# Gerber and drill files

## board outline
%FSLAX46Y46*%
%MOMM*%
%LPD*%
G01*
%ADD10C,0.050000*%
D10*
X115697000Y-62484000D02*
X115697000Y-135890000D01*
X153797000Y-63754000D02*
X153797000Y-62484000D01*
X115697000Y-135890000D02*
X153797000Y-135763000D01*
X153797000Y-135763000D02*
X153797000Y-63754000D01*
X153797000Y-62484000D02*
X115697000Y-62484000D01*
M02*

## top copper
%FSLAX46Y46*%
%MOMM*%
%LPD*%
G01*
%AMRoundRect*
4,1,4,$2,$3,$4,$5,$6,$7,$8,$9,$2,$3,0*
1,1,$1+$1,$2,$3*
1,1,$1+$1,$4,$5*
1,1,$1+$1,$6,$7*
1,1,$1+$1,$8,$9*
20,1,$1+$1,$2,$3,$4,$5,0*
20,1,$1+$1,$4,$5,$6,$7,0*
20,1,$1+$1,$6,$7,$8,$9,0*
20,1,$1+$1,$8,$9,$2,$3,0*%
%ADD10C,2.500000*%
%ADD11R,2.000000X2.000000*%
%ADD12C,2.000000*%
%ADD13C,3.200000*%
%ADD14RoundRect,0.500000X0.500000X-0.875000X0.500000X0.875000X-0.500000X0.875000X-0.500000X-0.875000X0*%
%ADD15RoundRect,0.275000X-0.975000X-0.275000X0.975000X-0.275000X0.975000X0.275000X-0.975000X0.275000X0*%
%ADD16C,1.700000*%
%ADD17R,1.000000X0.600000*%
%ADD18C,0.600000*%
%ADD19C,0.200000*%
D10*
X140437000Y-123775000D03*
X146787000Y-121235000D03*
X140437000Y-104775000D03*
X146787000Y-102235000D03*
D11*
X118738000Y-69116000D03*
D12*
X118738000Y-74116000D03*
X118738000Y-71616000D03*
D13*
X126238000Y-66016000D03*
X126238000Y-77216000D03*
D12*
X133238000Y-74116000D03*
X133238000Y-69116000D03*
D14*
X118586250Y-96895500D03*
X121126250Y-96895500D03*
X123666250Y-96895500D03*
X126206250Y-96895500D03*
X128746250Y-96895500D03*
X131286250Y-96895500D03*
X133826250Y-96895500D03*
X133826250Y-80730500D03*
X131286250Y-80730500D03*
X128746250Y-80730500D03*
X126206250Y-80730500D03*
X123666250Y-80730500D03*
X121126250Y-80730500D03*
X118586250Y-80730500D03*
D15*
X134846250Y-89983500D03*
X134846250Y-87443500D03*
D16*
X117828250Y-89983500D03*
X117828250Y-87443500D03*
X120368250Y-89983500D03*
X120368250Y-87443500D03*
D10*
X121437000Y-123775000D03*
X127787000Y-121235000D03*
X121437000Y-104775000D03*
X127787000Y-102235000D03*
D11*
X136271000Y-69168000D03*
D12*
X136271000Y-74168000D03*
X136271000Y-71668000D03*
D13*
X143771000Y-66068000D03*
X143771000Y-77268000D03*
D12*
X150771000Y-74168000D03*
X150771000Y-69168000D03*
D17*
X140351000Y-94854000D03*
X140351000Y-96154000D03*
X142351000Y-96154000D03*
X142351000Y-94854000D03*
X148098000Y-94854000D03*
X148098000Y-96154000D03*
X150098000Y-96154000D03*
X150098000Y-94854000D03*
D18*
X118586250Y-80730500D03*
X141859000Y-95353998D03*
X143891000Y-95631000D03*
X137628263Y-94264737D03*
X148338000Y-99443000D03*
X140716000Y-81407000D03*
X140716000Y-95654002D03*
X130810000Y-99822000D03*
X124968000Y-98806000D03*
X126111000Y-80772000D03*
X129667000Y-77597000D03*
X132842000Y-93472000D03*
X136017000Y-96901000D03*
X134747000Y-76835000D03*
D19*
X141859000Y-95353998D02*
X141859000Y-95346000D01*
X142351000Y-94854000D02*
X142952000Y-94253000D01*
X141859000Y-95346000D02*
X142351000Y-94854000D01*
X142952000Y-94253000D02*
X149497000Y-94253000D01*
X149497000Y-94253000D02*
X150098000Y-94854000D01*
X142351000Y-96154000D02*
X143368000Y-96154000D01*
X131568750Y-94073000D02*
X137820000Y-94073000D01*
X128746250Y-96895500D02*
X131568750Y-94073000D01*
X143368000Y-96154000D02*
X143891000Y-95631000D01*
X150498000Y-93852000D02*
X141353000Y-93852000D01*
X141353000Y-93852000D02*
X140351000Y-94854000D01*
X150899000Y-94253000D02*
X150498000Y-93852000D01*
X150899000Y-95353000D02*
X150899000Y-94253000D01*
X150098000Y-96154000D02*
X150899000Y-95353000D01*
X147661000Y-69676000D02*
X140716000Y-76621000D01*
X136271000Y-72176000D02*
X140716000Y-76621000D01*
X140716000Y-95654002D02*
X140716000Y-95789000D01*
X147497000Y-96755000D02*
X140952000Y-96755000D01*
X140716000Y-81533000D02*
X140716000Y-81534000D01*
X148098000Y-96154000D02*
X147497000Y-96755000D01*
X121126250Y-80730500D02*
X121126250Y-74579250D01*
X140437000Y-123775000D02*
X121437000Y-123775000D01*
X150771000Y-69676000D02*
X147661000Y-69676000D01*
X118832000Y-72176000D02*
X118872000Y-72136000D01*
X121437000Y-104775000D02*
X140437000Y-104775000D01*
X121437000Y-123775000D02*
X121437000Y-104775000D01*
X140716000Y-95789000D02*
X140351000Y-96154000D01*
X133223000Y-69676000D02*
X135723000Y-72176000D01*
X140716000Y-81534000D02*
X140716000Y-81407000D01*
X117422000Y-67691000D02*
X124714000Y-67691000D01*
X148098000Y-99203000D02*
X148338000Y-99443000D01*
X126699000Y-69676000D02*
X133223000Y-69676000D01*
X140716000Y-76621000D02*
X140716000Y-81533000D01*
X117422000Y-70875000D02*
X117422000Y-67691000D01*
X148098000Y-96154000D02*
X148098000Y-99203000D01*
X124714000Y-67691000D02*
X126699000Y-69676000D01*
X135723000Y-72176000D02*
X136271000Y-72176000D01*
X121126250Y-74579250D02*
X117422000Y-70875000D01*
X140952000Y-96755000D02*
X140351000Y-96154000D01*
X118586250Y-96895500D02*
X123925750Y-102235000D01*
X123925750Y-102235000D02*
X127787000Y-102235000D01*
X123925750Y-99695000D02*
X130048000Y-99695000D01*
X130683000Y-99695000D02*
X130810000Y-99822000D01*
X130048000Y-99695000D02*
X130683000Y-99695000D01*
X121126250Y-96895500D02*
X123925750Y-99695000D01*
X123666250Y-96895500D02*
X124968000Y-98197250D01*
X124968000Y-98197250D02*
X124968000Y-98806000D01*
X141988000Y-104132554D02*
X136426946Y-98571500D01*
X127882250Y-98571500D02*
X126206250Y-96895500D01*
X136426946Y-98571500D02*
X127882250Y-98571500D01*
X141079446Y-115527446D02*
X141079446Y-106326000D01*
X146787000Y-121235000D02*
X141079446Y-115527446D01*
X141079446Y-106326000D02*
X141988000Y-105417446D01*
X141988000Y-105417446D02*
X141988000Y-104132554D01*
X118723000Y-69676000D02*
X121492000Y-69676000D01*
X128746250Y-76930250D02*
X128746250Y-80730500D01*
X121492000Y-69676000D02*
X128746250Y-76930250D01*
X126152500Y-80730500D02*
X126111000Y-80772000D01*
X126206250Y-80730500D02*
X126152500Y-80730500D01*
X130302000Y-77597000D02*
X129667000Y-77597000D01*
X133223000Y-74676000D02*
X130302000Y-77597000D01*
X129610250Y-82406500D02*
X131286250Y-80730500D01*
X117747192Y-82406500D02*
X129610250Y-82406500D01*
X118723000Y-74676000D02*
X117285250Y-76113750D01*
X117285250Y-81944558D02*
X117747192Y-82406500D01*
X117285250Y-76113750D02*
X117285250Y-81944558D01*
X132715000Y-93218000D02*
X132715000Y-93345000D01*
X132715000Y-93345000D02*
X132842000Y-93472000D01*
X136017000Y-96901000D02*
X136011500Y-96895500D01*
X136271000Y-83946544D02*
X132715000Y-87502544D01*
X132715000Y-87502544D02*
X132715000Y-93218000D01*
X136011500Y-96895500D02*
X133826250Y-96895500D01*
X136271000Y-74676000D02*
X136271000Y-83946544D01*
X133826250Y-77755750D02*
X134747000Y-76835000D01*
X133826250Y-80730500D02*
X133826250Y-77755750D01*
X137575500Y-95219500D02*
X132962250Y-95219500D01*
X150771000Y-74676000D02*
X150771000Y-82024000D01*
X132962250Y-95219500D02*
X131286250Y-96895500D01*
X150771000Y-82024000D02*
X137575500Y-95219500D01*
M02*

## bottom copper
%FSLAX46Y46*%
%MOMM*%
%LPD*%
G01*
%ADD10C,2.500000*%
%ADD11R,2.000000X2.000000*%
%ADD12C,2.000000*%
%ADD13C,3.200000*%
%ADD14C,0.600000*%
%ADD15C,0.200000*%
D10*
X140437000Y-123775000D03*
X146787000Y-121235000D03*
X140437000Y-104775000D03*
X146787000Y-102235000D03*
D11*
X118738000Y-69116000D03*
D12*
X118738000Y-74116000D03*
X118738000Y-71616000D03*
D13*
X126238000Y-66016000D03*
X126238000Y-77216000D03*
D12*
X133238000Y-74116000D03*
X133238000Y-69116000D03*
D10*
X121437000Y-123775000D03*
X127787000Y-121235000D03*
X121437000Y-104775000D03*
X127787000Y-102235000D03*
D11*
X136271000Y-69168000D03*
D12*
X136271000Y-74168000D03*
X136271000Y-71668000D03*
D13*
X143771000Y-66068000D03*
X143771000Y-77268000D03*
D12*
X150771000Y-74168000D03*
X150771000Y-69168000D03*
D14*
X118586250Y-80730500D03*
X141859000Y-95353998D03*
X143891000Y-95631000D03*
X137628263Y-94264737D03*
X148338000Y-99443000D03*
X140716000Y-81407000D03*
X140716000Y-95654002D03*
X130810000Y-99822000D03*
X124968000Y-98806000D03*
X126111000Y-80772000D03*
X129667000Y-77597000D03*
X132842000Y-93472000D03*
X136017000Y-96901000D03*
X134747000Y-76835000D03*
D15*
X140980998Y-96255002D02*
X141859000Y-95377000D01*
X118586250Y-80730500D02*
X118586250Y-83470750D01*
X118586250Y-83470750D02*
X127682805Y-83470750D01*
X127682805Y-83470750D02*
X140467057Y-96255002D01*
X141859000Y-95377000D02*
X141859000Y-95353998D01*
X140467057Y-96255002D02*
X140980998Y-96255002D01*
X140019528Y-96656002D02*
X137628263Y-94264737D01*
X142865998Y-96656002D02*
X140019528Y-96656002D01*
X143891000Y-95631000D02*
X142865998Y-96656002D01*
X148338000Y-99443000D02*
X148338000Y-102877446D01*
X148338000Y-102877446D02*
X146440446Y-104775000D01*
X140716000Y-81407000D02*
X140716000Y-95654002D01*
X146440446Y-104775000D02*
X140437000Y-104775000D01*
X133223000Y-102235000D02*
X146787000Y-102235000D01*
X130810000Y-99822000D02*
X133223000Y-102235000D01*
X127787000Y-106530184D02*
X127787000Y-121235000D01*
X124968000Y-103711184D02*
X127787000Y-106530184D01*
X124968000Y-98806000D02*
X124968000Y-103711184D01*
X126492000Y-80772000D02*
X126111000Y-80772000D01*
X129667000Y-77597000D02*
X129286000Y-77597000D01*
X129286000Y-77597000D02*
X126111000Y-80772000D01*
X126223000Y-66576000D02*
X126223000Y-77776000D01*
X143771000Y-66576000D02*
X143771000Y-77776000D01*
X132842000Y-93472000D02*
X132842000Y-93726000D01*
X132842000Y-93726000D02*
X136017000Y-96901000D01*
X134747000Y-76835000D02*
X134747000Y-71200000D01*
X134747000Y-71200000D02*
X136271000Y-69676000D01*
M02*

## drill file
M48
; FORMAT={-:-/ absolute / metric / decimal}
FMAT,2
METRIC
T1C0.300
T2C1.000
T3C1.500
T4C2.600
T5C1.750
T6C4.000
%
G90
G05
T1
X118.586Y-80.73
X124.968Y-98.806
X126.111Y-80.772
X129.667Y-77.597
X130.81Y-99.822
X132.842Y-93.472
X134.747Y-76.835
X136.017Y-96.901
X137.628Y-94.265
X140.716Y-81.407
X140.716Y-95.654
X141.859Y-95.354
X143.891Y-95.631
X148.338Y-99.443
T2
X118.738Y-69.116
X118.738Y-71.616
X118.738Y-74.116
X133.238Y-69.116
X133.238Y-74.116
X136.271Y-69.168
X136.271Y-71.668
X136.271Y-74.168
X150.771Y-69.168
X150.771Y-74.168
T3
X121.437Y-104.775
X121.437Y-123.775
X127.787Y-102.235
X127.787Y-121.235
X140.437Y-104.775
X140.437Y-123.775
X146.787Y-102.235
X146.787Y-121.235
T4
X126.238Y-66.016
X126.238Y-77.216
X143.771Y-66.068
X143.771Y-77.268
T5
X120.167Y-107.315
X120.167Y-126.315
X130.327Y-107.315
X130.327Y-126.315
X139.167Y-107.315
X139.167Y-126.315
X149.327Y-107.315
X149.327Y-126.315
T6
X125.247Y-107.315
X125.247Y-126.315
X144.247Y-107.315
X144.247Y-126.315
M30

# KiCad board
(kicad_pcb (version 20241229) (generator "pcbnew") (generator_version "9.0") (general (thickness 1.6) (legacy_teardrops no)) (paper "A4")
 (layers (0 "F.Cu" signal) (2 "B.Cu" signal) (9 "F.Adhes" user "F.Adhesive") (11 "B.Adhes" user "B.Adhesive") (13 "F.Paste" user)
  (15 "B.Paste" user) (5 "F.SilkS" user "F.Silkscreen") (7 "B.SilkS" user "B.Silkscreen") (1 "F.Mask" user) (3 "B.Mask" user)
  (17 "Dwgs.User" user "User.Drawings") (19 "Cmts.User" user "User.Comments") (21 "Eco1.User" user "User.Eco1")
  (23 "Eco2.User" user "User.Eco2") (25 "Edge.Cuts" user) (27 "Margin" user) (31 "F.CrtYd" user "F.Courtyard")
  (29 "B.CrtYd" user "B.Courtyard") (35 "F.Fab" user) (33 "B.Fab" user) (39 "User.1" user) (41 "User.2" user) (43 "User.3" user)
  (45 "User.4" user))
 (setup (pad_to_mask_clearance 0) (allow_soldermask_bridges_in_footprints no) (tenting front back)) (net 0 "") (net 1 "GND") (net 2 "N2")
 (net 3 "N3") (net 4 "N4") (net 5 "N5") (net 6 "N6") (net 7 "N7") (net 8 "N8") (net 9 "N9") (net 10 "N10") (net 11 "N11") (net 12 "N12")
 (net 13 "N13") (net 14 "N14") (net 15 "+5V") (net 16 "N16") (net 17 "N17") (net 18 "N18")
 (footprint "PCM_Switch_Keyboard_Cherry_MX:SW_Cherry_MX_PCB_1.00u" (layer "F.Cu") (at 144.247 126.315)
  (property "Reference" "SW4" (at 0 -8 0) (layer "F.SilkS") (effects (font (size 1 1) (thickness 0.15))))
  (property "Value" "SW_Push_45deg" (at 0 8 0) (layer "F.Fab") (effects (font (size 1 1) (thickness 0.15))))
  (pad "" np_thru_hole circle (at -5.08 0) (size 1.75 1.75) (drill 1.75) (layers "*.Cu" "*.Mask"))
  (pad "" np_thru_hole circle (at 0 0) (size 4 4) (drill 4) (layers "*.Cu" "*.Mask"))
  (pad "" np_thru_hole circle (at 5.08 0) (size 1.75 1.75) (drill 1.75) (layers "*.Cu" "*.Mask"))
  (pad "1" thru_hole circle (at -3.81 -2.54) (size 2.5 2.5) (drill 1.5) (layers "*.Cu" "*.Mask") (remove_unused_layers no) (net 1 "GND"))
  (pad "2" thru_hole circle (at 2.54 -5.08) (size 2.5 2.5) (drill 1.5) (layers "*.Cu" "*.Mask") (remove_unused_layers no) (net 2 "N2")))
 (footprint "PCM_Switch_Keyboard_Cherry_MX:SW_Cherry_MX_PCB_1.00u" (layer "F.Cu") (at 144.247 107.315)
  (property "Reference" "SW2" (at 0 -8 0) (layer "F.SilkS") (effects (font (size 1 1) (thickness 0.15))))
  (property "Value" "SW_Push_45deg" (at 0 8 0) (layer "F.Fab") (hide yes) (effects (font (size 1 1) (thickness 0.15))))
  (pad "" np_thru_hole circle (at -5.08 0) (size 1.75 1.75) (drill 1.75) (layers "*.Cu" "*.Mask"))
  (pad "" np_thru_hole circle (at 0 0) (size 4 4) (drill 4) (layers "*.Cu" "*.Mask"))
  (pad "" np_thru_hole circle (at 5.08 0) (size 1.75 1.75) (drill 1.75) (layers "*.Cu" "*.Mask"))
  (pad "1" thru_hole circle (at -3.81 -2.54) (size 2.5 2.5) (drill 1.5) (layers "*.Cu" "*.Mask") (remove_unused_layers no) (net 1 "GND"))
  (pad "2" thru_hole circle (at 2.54 -5.08) (size 2.5 2.5) (drill 1.5) (layers "*.Cu" "*.Mask") (remove_unused_layers no) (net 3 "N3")))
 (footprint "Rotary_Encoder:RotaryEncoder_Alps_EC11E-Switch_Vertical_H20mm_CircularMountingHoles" (layer "F.Cu") (at 118.738 69.116)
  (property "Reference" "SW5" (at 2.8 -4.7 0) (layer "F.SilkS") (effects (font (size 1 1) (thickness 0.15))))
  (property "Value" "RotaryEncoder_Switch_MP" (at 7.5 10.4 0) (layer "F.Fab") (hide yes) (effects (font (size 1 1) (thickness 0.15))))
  (pad "A" thru_hole rect (at 0 0) (size 2 2) (drill 1) (layers "*.Cu" "*.Mask") (remove_unused_layers no) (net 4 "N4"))
  (pad "B" thru_hole circle (at 0 5) (size 2 2) (drill 1) (layers "*.Cu" "*.Mask") (remove_unused_layers no) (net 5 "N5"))
  (pad "C" thru_hole circle (at 0 2.5) (size 2 2) (drill 1) (layers "*.Cu" "*.Mask") (remove_unused_layers no) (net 1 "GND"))
  (pad "MP" thru_hole circle (at 7.5 -3.1) (size 3.2 3.2) (drill 2.6) (layers "*.Cu" "*.Mask") (remove_unused_layers no) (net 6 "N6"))
  (pad "MP" thru_hole circle (at 7.5 8.1) (size 3.2 3.2) (drill 2.6) (layers "*.Cu" "*.Mask") (remove_unused_layers no) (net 6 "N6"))
  (pad "S1" thru_hole circle (at 14.5 5) (size 2 2) (drill 1) (layers "*.Cu" "*.Mask") (remove_unused_layers no) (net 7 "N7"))
  (pad "S2" thru_hole circle (at 14.5 0) (size 2 2) (drill 1) (layers "*.Cu" "*.Mask") (remove_unused_layers no) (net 1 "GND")))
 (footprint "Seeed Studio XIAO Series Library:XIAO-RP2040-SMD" (layer "F.Cu") (at 126.20625 88.8955 90)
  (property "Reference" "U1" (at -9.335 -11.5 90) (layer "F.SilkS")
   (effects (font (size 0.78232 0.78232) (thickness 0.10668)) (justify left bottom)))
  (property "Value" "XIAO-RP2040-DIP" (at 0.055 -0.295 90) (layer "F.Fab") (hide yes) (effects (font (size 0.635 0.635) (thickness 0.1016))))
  (pad "1" smd roundrect (at -8 -7.62 90) (size 2.75 2) (layers "F.Cu" "F.Mask" "F.Paste") (roundrect_rratio 0.25) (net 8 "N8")
   (solder_mask_margin 0.0508) (thermal_bridge_angle 45))
  (pad "2" smd roundrect (at -8 -5.08 90) (size 2.75 2) (layers "F.Cu" "F.Mask" "F.Paste") (roundrect_rratio 0.25) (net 3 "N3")
   (solder_mask_margin 0.0508) (thermal_bridge_angle 45))
  (pad "3" smd roundrect (at -8 -2.54 90) (size 2.75 2) (layers "F.Cu" "F.Mask" "F.Paste") (roundrect_rratio 0.25) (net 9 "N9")
   (solder_mask_margin 0.0508) (thermal_bridge_angle 45))
  (pad "4" smd roundrect (at -8 0 90) (size 2.75 2) (layers "F.Cu" "F.Mask" "F.Paste") (roundrect_rratio 0.25) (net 2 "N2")
   (solder_mask_margin 0.0508) (thermal_bridge_angle 45))
  (pad "5" smd roundrect (at -8 2.54 90) (size 2.75 2) (layers "F.Cu" "F.Mask" "F.Paste") (roundrect_rratio 0.25) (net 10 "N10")
   (solder_mask_margin 0.0508) (thermal_bridge_angle 45))
  (pad "6" smd roundrect (at -8 5.08 90) (size 2.75 2) (layers "F.Cu" "F.Mask" "F.Paste") (roundrect_rratio 0.25) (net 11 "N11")
   (solder_mask_margin 0.0508) (thermal_bridge_angle 45))
  (pad "7" smd roundrect (at -8 7.62 90) (size 2.75 2) (layers "F.Cu" "F.Mask" "F.Paste") (roundrect_rratio 0.25) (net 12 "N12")
   (solder_mask_margin 0.0508) (thermal_bridge_angle 45))
  (pad "8" smd roundrect (at 8.165 7.62 90) (size 2.75 2) (layers "F.Cu" "F.Mask" "F.Paste") (roundrect_rratio 0.25) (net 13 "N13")
   (solder_mask_margin 0.0508) (thermal_bridge_angle 45))
  (pad "9" smd roundrect (at 8.165 5.08 90) (size 2.75 2) (layers "F.Cu" "F.Mask" "F.Paste") (roundrect_rratio 0.25) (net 5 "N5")
   (solder_mask_margin 0.0508) (thermal_bridge_angle 45))
  (pad "10" smd roundrect (at 8.165 2.54 90) (size 2.75 2) (layers "F.Cu" "F.Mask" "F.Paste") (roundrect_rratio 0.25) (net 4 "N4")
   (solder_mask_margin 0.0508) (thermal_bridge_angle 45))
  (pad "11" smd roundrect (at 8.165 0 90) (size 2.75 2) (layers "F.Cu" "F.Mask" "F.Paste") (roundrect_rratio 0.25) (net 7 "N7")
   (solder_mask_margin 0.0508) (thermal_bridge_angle 45))
  (pad "12" smd roundrect (at 8.165 -2.54 90) (size 2.75 2) (layers "F.Cu" "F.Mask" "F.Paste") (roundrect_rratio 0.25) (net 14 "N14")
   (solder_mask_margin 0.0508) (thermal_bridge_angle 45))
  (pad "13" smd roundrect (at 8.165 -5.08 90) (size 2.75 2) (layers "F.Cu" "F.Mask" "F.Paste") (roundrect_rratio 0.25) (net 1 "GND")
   (solder_mask_margin 0.0508) (thermal_bridge_angle 45))
  (pad "14" smd roundrect (at 8.165 -7.62 90) (size 2.75 2) (layers "F.Cu" "F.Mask" "F.Paste") (roundrect_rratio 0.25) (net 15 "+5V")
   (solder_mask_margin 0.0508) (thermal_bridge_angle 45))
  (pad "15" smd roundrect (at -1.088 8.64) (size 2.5 1.1) (layers "F.Cu" "F.Mask" "F.Paste") (roundrect_rratio 0.25)
   (thermal_bridge_angle 45))
  (pad "16" smd roundrect (at 1.452 8.64) (size 2.5 1.1) (layers "F.Cu" "F.Mask" "F.Paste") (roundrect_rratio 0.25)
   (thermal_bridge_angle 45))
  (pad "17" smd circle (at -1.088 -8.378 90) (size 1.7 1.7) (layers "F.Cu" "F.Mask" "F.Paste"))
  (pad "18" smd circle (at 1.452 -8.378 90) (size 1.7 1.7) (layers "F.Cu" "F.Mask" "F.Paste"))
  (pad "19" smd circle (at -1.088 -5.838 90) (size 1.7 1.7) (layers "F.Cu" "F.Mask" "F.Paste"))
  (pad "20" smd circle (at 1.452 -5.838 90) (size 1.7 1.7) (layers "F.Cu" "F.Mask" "F.Paste")))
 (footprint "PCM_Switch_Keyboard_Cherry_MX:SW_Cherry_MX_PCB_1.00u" (layer "F.Cu") (at 125.247 126.315)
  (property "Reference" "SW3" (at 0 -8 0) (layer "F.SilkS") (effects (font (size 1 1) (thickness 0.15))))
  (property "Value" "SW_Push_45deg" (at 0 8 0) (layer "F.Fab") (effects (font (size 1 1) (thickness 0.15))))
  (pad "" np_thru_hole circle (at -5.08 0) (size 1.75 1.75) (drill 1.75) (layers "*.Cu" "*.Mask"))
  (pad "" np_thru_hole circle (at 0 0) (size 4 4) (drill 4) (layers "*.Cu" "*.Mask"))
  (pad "" np_thru_hole circle (at 5.08 0) (size 1.75 1.75) (drill 1.75) (layers "*.Cu" "*.Mask"))
  (pad "1" thru_hole circle (at -3.81 -2.54) (size 2.5 2.5) (drill 1.5) (layers "*.Cu" "*.Mask") (remove_unused_layers no) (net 1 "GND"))
  (pad "2" thru_hole circle (at 2.54 -5.08) (size 2.5 2.5) (drill 1.5) (layers "*.Cu" "*.Mask") (remove_unused_layers no) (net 9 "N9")))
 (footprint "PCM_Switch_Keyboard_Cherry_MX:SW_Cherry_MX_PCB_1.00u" (layer "F.Cu") (at 125.247 107.315)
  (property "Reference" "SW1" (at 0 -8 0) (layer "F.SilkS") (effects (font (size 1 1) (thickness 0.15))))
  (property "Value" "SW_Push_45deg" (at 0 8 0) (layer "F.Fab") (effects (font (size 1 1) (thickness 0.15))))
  (pad "" np_thru_hole circle (at -5.08 0) (size 1.75 1.75) (drill 1.75) (layers "*.Cu" "*.Mask"))
  (pad "" np_thru_hole circle (at 0 0) (size 4 4) (drill 4) (layers "*.Cu" "*.Mask"))
  (pad "" np_thru_hole circle (at 5.08 0) (size 1.75 1.75) (drill 1.75) (layers "*.Cu" "*.Mask"))
  (pad "1" thru_hole circle (at -3.81 -2.54) (size 2.5 2.5) (drill 1.5) (layers "*.Cu" "*.Mask") (remove_unused_layers no) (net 1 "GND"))
  (pad "2" thru_hole circle (at 2.54 -5.08) (size 2.5 2.5) (drill 1.5) (layers "*.Cu" "*.Mask") (remove_unused_layers no) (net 8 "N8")))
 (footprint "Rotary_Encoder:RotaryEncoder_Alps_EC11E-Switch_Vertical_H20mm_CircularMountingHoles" (layer "F.Cu") (at 136.271 69.168)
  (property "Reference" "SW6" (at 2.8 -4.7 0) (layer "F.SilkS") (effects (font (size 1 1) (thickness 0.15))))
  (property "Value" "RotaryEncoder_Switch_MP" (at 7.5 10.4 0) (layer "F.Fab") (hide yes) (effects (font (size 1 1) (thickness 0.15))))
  (pad "A" thru_hole rect (at 0 0) (size 2 2) (drill 1) (layers "*.Cu" "*.Mask") (remove_unused_layers no) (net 13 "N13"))
  (pad "B" thru_hole circle (at 0 5) (size 2 2) (drill 1) (layers "*.Cu" "*.Mask") (remove_unused_layers no) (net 12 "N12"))
  (pad "C" thru_hole circle (at 0 2.5) (size 2 2) (drill 1) (layers "*.Cu" "*.Mask") (remove_unused_layers no) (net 1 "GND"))
  (pad "MP" thru_hole circle (at 7.5 -3.1) (size 3.2 3.2) (drill 2.6) (layers "*.Cu" "*.Mask") (remove_unused_layers no) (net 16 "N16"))
  (pad "MP" thru_hole circle (at 7.5 8.1) (size 3.2 3.2) (drill 2.6) (layers "*.Cu" "*.Mask") (remove_unused_layers no) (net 16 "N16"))
  (pad "S1" thru_hole circle (at 14.5 5) (size 2 2) (drill 1) (layers "*.Cu" "*.Mask") (remove_unused_layers no) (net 11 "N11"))
  (pad "S2" thru_hole circle (at 14.5 0) (size 2 2) (drill 1) (layers "*.Cu" "*.Mask") (remove_unused_layers no) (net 1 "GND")))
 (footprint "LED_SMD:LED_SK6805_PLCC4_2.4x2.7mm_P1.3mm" (layer "F.Cu") (at 141.351 95.504)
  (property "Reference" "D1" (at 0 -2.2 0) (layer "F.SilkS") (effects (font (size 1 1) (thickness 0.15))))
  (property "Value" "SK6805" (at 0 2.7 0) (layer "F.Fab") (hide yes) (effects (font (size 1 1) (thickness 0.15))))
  (pad "1" smd rect (at -1 -0.65) (size 1 0.6) (layers "F.Cu" "F.Mask" "F.Paste") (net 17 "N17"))
  (pad "2" smd rect (at -1 0.65) (size 1 0.6) (layers "F.Cu" "F.Mask" "F.Paste") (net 1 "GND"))
  (pad "3" smd rect (at 1 0.65) (size 1 0.6) (layers "F.Cu" "F.Mask" "F.Paste") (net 10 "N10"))
  (pad "4" smd rect (at 1 -0.65) (size 1 0.6) (layers "F.Cu" "F.Mask" "F.Paste") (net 15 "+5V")))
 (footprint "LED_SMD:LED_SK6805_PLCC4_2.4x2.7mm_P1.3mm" (layer "F.Cu") (at 149.098 95.504)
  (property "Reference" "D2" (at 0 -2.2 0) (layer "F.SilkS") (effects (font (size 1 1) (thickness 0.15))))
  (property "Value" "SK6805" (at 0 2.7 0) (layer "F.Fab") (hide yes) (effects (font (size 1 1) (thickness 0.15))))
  (pad "1" smd rect (at -1 -0.65) (size 1 0.6) (layers "F.Cu" "F.Mask" "F.Paste") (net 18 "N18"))
  (pad "2" smd rect (at -1 0.65) (size 1 0.6) (layers "F.Cu" "F.Mask" "F.Paste") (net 1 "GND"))
  (pad "3" smd rect (at 1 0.65) (size 1 0.6) (layers "F.Cu" "F.Mask" "F.Paste") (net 17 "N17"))
  (pad "4" smd rect (at 1 -0.65) (size 1 0.6) (layers "F.Cu" "F.Mask" "F.Paste") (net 15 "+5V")))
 (gr_line (start 115.697 62.484) (end 115.697 135.89) (stroke (width 0.05) (type default)) (layer "Edge.Cuts"))
 (gr_line (start 153.797 63.754) (end 153.797 62.484) (stroke (width 0.05) (type default)) (layer "Edge.Cuts"))
 (gr_line (start 115.697 135.89) (end 153.797 135.763) (stroke (width 0.05) (type default)) (layer "Edge.Cuts"))
 (gr_line (start 153.797 135.763) (end 153.797 63.754) (stroke (width 0.05) (type default)) (layer "Edge.Cuts"))
 (gr_line (start 153.797 62.484) (end 115.697 62.484) (stroke (width 0.05) (type default)) (layer "Edge.Cuts"))
 (segment (start 141.859 95.353998) (end 141.859 95.346) (width 0.2) (layer "F.Cu") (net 15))
 (segment (start 142.351 94.854) (end 142.952 94.253) (width 0.2) (layer "F.Cu") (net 15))
 (segment (start 141.859 95.346) (end 142.351 94.854) (width 0.2) (layer "F.Cu") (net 15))
 (segment (start 142.952 94.253) (end 149.497 94.253) (width 0.2) (layer "F.Cu") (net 15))
 (segment (start 149.497 94.253) (end 150.098 94.854) (width 0.2) (layer "F.Cu") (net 15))
 (via (at 118.58625 80.7305) (size 0.6) (drill 0.3) (layers "F.Cu" "B.Cu") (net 15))
 (via (at 141.859 95.353998) (size 0.6) (drill 0.3) (layers "F.Cu" "B.Cu") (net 15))
 (segment (start 140.980998 96.255002) (end 141.859 95.377) (width 0.2) (layer "B.Cu") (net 15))
 (segment (start 118.58625 80.7305) (end 118.58625 83.47075) (width 0.2) (layer "B.Cu") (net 15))
 (segment (start 118.58625 83.47075) (end 127.682805 83.47075) (width 0.2) (layer "B.Cu") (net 15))
 (segment (start 127.682805 83.47075) (end 140.467057 96.255002) (width 0.2) (layer "B.Cu") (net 15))
 (segment (start 141.859 95.377) (end 141.859 95.353998) (width 0.2) (layer "B.Cu") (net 15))
 (segment (start 140.467057 96.255002) (end 140.980998 96.255002) (width 0.2) (layer "B.Cu") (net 15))
 (segment (start 142.351 96.154) (end 143.368 96.154) (width 0.2) (layer "F.Cu") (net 10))
 (segment (start 131.56875 94.073) (end 137.82 94.073) (width 0.2) (layer "F.Cu") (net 10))
 (segment (start 128.74625 96.8955) (end 131.56875 94.073) (width 0.2) (layer "F.Cu") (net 10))
 (segment (start 143.368 96.154) (end 143.891 95.631) (width 0.2) (layer "F.Cu") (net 10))
 (via (at 143.891 95.631) (size 0.6) (drill 0.3) (layers "F.Cu" "B.Cu") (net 10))
 (via (at 137.628263 94.264737) (size 0.6) (drill 0.3) (layers "F.Cu" "B.Cu") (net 10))
 (segment (start 140.019528 96.656002) (end 137.628263 94.264737) (width 0.2) (layer "B.Cu") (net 10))
 (segment (start 142.865998 96.656002) (end 140.019528 96.656002) (width 0.2) (layer "B.Cu") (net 10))
 (segment (start 143.891 95.631) (end 142.865998 96.656002) (width 0.2) (layer "B.Cu") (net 10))
 (segment (start 150.498 93.852) (end 141.353 93.852) (width 0.2) (layer "F.Cu") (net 17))
 (segment (start 141.353 93.852) (end 140.351 94.854) (width 0.2) (layer "F.Cu") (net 17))
 (segment (start 150.899 94.253) (end 150.498 93.852) (width 0.2) (layer "F.Cu") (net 17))
 (segment (start 150.899 95.353) (end 150.899 94.253) (width 0.2) (layer "F.Cu") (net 17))
 (segment (start 150.098 96.154) (end 150.899 95.353) (width 0.2) (layer "F.Cu") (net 17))
 (segment (start 147.661 69.676) (end 140.716 76.621) (width 0.2) (layer "F.Cu") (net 1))
 (segment (start 136.271 72.176) (end 140.716 76.621) (width 0.2) (layer "F.Cu") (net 1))
 (segment (start 140.716 95.654002) (end 140.716 95.789) (width 0.2) (layer "F.Cu") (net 1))
 (segment (start 147.497 96.755) (end 140.952 96.755) (width 0.2) (layer "F.Cu") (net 1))
 (segment (start 140.716 81.533) (end 140.716 81.534) (width 0.2) (layer "F.Cu") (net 1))
 (segment (start 148.098 96.154) (end 147.497 96.755) (width 0.2) (layer "F.Cu") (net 1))
 (segment (start 121.12625 80.7305) (end 121.12625 74.57925) (width 0.2) (layer "F.Cu") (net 1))
 (segment (start 140.437 123.775) (end 121.437 123.775) (width 0.2) (layer "F.Cu") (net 1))
 (segment (start 150.771 69.676) (end 147.661 69.676) (width 0.2) (layer "F.Cu") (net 1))
 (segment (start 118.832 72.176) (end 118.872 72.136) (width 0.2) (layer "F.Cu") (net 1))
 (segment (start 121.437 104.775) (end 140.437 104.775) (width 0.2) (layer "F.Cu") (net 1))
 (segment (start 121.437 123.775) (end 121.437 104.775) (width 0.2) (layer "F.Cu") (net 1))
 (segment (start 140.716 95.789) (end 140.351 96.154) (width 0.2) (layer "F.Cu") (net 1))
 (segment (start 133.223 69.676) (end 135.723 72.176) (width 0.2) (layer "F.Cu") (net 1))
 (segment (start 140.716 81.534) (end 140.716 81.407) (width 0.2) (layer "F.Cu") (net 1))
 (segment (start 117.422 67.691) (end 124.714 67.691) (width 0.2) (layer "F.Cu") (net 1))
 (segment (start 148.098 99.203) (end 148.338 99.443) (width 0.2) (layer "F.Cu") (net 1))
 (segment (start 126.699 69.676) (end 133.223 69.676) (width 0.2) (layer "F.Cu") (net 1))
 (segment (start 140.716 76.621) (end 140.716 81.533) (width 0.2) (layer "F.Cu") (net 1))
 (segment (start 117.422 70.875) (end 117.422 67.691) (width 0.2) (layer "F.Cu") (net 1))
 (segment (start 148.098 96.154) (end 148.098 99.203) (width 0.2) (layer "F.Cu") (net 1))
 (segment (start 124.714 67.691) (end 126.699 69.676) (width 0.2) (layer "F.Cu") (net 1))
 (segment (start 135.723 72.176) (end 136.271 72.176) (width 0.2) (layer "F.Cu") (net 1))
 (segment (start 121.12625 74.57925) (end 117.422 70.875) (width 0.2) (layer "F.Cu") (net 1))
 (segment (start 140.952 96.755) (end 140.351 96.154) (width 0.2) (layer "F.Cu") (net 1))
 (via (at 148.338 99.443) (size 0.6) (drill 0.3) (layers "F.Cu" "B.Cu") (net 1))
 (via (at 140.716 81.407) (size 0.6) (drill 0.3) (layers "F.Cu" "B.Cu") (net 1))
 (via (at 140.716 95.654002) (size 0.6) (drill 0.3) (layers "F.Cu" "B.Cu") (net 1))
 (segment (start 148.338 99.443) (end 148.338 102.877446) (width 0.2) (layer "B.Cu") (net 1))
 (segment (start 148.338 102.877446) (end 146.440446 104.775) (width 0.2) (layer "B.Cu") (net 1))
 (segment (start 140.716 81.407) (end 140.716 95.654002) (width 0.2) (layer "B.Cu") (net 1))
 (segment (start 146.440446 104.775) (end 140.437 104.775) (width 0.2) (layer "B.Cu") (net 1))
 (segment (start 118.58625 96.8955) (end 123.92575 102.235) (width 0.2) (layer "F.Cu") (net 8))
 (segment (start 123.92575 102.235) (end 127.787 102.235) (width 0.2) (layer "F.Cu") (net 8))
 (segment (start 123.92575 99.695) (end 130.048 99.695) (width 0.2) (layer "F.Cu") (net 3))
 (segment (start 130.683 99.695) (end 130.81 99.822) (width 0.2) (layer "F.Cu") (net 3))
 (segment (start 130.048 99.695) (end 130.683 99.695) (width 0.2) (layer "F.Cu") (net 3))
 (segment (start 121.12625 96.8955) (end 123.92575 99.695) (width 0.2) (layer "F.Cu") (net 3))
 (via (at 130.81 99.822) (size 0.6) (drill 0.3) (layers "F.Cu" "B.Cu") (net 3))
 (segment (start 133.223 102.235) (end 146.787 102.235) (width 0.2) (layer "B.Cu") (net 3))
 (segment (start 130.81 99.822) (end 133.223 102.235) (width 0.2) (layer "B.Cu") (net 3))
 (segment (start 123.66625 96.8955) (end 124.968 98.19725) (width 0.2) (layer "F.Cu") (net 9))
 (segment (start 124.968 98.19725) (end 124.968 98.806) (width 0.2) (layer "F.Cu") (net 9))
 (via (at 124.968 98.806) (size 0.6) (drill 0.3) (layers "F.Cu" "B.Cu") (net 9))
 (segment (start 127.787 106.530184) (end 127.787 121.235) (width 0.2) (layer "B.Cu") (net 9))
 (segment (start 124.968 103.711184) (end 127.787 106.530184) (width 0.2) (layer "B.Cu") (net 9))
 (segment (start 124.968 98.806) (end 124.968 103.711184) (width 0.2) (layer "B.Cu") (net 9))
 (segment (start 141.988 104.132554) (end 136.426946 98.5715) (width 0.2) (layer "F.Cu") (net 2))
 (segment (start 127.88225 98.5715) (end 126.20625 96.8955) (width 0.2) (layer "F.Cu") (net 2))
 (segment (start 136.426946 98.5715) (end 127.88225 98.5715) (width 0.2) (layer "F.Cu") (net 2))
 (segment (start 141.079446 115.527446) (end 141.079446 106.326) (width 0.2) (layer "F.Cu") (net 2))
 (segment (start 146.787 121.235) (end 141.079446 115.527446) (width 0.2) (layer "F.Cu") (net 2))
 (segment (start 141.079446 106.326) (end 141.988 105.417446) (width 0.2) (layer "F.Cu") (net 2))
 (segment (start 141.988 105.417446) (end 141.988 104.132554) (width 0.2) (layer "F.Cu") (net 2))
 (segment (start 118.723 69.676) (end 121.492 69.676) (width 0.2) (layer "F.Cu") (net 4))
 (segment (start 128.74625 76.93025) (end 128.74625 80.7305) (width 0.2) (layer "F.Cu") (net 4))
 (segment (start 121.492 69.676) (end 128.74625 76.93025) (width 0.2) (layer "F.Cu") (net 4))
 (segment (start 126.1525 80.7305) (end 126.111 80.772) (width 0.2) (layer "F.Cu") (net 7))
 (segment (start 126.20625 80.7305) (end 126.1525 80.7305) (width 0.2) (layer "F.Cu") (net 7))
 (segment (start 130.302 77.597) (end 129.667 77.597) (width 0.2) (layer "F.Cu") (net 7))
 (segment (start 133.223 74.676) (end 130.302 77.597) (width 0.2) (layer "F.Cu") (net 7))
 (via (at 126.111 80.772) (size 0.6) (drill 0.3) (layers "F.Cu" "B.Cu") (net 7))
 (via (at 129.667 77.597) (size 0.6) (drill 0.3) (layers "F.Cu" "B.Cu") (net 7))
 (segment (start 126.492 80.772) (end 126.111 80.772) (width 0.2) (layer "B.Cu") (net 7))
 (segment (start 129.667 77.597) (end 129.286 77.597) (width 0.2) (layer "B.Cu") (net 7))
 (segment (start 129.286 77.597) (end 126.111 80.772) (width 0.2) (layer "B.Cu") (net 7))
 (segment (start 129.61025 82.4065) (end 131.28625 80.7305) (width 0.2) (layer "F.Cu") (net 5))
 (segment (start 117.747192 82.4065) (end 129.61025 82.4065) (width 0.2) (layer "F.Cu") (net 5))
 (segment (start 118.723 74.676) (end 117.28525 76.11375) (width 0.2) (layer "F.Cu") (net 5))
 (segment (start 117.28525 81.944558) (end 117.747192 82.4065) (width 0.2) (layer "F.Cu") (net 5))
 (segment (start 117.28525 76.11375) (end 117.28525 81.944558) (width 0.2) (layer "F.Cu") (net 5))
 (segment (start 126.223 66.576) (end 126.223 77.776) (width 0.2) (layer "B.Cu") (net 6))
 (segment (start 143.771 66.576) (end 143.771 77.776) (width 0.2) (layer "B.Cu") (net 16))
 (segment (start 132.715 93.218) (end 132.715 93.345) (width 0.2) (layer "F.Cu") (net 12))
 (segment (start 132.715 93.345) (end 132.842 93.472) (width 0.2) (layer "F.Cu") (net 12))
 (segment (start 136.017 96.901) (end 136.0115 96.8955) (width 0.2) (layer "F.Cu") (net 12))
 (segment (start 136.271 83.946544) (end 132.715 87.502544) (width 0.2) (layer "F.Cu") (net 12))
 (segment (start 132.715 87.502544) (end 132.715 93.218) (width 0.2) (layer "F.Cu") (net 12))
 (segment (start 136.0115 96.8955) (end 133.82625 96.8955) (width 0.2) (layer "F.Cu") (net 12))
 (segment (start 136.271 74.676) (end 136.271 83.946544) (width 0.2) (layer "F.Cu") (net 12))
 (via (at 132.842 93.472) (size 0.6) (drill 0.3) (layers "F.Cu" "B.Cu") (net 12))
 (via (at 136.017 96.901) (size 0.6) (drill 0.3) (layers "F.Cu" "B.Cu") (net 12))
 (segment (start 132.842 93.472) (end 132.842 93.726) (width 0.2) (layer "B.Cu") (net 12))
 (segment (start 132.842 93.726) (end 136.017 96.901) (width 0.2) (layer "B.Cu") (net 12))
 (segment (start 133.82625 77.75575) (end 134.747 76.835) (width 0.2) (layer "F.Cu") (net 13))
 (segment (start 133.82625 80.7305) (end 133.82625 77.75575) (width 0.2) (layer "F.Cu") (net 13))
 (via (at 134.747 76.835) (size 0.6) (drill 0.3) (layers "F.Cu" "B.Cu") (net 13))
 (segment (start 134.747 76.835) (end 134.747 71.2) (width 0.2) (layer "B.Cu") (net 13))
 (segment (start 134.747 71.2) (end 136.271 69.676) (width 0.2) (layer "B.Cu") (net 13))
 (segment (start 137.5755 95.2195) (end 132.96225 95.2195) (width 0.2) (layer "F.Cu") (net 11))
 (segment (start 150.771 74.676) (end 150.771 82.024) (width 0.2) (layer "F.Cu") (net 11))
 (segment (start 132.96225 95.2195) (end 131.28625 96.8955) (width 0.2) (layer "F.Cu") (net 11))
 (segment (start 150.771 82.024) (end 137.5755 95.2195) (width 0.2) (layer "F.Cu") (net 11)))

